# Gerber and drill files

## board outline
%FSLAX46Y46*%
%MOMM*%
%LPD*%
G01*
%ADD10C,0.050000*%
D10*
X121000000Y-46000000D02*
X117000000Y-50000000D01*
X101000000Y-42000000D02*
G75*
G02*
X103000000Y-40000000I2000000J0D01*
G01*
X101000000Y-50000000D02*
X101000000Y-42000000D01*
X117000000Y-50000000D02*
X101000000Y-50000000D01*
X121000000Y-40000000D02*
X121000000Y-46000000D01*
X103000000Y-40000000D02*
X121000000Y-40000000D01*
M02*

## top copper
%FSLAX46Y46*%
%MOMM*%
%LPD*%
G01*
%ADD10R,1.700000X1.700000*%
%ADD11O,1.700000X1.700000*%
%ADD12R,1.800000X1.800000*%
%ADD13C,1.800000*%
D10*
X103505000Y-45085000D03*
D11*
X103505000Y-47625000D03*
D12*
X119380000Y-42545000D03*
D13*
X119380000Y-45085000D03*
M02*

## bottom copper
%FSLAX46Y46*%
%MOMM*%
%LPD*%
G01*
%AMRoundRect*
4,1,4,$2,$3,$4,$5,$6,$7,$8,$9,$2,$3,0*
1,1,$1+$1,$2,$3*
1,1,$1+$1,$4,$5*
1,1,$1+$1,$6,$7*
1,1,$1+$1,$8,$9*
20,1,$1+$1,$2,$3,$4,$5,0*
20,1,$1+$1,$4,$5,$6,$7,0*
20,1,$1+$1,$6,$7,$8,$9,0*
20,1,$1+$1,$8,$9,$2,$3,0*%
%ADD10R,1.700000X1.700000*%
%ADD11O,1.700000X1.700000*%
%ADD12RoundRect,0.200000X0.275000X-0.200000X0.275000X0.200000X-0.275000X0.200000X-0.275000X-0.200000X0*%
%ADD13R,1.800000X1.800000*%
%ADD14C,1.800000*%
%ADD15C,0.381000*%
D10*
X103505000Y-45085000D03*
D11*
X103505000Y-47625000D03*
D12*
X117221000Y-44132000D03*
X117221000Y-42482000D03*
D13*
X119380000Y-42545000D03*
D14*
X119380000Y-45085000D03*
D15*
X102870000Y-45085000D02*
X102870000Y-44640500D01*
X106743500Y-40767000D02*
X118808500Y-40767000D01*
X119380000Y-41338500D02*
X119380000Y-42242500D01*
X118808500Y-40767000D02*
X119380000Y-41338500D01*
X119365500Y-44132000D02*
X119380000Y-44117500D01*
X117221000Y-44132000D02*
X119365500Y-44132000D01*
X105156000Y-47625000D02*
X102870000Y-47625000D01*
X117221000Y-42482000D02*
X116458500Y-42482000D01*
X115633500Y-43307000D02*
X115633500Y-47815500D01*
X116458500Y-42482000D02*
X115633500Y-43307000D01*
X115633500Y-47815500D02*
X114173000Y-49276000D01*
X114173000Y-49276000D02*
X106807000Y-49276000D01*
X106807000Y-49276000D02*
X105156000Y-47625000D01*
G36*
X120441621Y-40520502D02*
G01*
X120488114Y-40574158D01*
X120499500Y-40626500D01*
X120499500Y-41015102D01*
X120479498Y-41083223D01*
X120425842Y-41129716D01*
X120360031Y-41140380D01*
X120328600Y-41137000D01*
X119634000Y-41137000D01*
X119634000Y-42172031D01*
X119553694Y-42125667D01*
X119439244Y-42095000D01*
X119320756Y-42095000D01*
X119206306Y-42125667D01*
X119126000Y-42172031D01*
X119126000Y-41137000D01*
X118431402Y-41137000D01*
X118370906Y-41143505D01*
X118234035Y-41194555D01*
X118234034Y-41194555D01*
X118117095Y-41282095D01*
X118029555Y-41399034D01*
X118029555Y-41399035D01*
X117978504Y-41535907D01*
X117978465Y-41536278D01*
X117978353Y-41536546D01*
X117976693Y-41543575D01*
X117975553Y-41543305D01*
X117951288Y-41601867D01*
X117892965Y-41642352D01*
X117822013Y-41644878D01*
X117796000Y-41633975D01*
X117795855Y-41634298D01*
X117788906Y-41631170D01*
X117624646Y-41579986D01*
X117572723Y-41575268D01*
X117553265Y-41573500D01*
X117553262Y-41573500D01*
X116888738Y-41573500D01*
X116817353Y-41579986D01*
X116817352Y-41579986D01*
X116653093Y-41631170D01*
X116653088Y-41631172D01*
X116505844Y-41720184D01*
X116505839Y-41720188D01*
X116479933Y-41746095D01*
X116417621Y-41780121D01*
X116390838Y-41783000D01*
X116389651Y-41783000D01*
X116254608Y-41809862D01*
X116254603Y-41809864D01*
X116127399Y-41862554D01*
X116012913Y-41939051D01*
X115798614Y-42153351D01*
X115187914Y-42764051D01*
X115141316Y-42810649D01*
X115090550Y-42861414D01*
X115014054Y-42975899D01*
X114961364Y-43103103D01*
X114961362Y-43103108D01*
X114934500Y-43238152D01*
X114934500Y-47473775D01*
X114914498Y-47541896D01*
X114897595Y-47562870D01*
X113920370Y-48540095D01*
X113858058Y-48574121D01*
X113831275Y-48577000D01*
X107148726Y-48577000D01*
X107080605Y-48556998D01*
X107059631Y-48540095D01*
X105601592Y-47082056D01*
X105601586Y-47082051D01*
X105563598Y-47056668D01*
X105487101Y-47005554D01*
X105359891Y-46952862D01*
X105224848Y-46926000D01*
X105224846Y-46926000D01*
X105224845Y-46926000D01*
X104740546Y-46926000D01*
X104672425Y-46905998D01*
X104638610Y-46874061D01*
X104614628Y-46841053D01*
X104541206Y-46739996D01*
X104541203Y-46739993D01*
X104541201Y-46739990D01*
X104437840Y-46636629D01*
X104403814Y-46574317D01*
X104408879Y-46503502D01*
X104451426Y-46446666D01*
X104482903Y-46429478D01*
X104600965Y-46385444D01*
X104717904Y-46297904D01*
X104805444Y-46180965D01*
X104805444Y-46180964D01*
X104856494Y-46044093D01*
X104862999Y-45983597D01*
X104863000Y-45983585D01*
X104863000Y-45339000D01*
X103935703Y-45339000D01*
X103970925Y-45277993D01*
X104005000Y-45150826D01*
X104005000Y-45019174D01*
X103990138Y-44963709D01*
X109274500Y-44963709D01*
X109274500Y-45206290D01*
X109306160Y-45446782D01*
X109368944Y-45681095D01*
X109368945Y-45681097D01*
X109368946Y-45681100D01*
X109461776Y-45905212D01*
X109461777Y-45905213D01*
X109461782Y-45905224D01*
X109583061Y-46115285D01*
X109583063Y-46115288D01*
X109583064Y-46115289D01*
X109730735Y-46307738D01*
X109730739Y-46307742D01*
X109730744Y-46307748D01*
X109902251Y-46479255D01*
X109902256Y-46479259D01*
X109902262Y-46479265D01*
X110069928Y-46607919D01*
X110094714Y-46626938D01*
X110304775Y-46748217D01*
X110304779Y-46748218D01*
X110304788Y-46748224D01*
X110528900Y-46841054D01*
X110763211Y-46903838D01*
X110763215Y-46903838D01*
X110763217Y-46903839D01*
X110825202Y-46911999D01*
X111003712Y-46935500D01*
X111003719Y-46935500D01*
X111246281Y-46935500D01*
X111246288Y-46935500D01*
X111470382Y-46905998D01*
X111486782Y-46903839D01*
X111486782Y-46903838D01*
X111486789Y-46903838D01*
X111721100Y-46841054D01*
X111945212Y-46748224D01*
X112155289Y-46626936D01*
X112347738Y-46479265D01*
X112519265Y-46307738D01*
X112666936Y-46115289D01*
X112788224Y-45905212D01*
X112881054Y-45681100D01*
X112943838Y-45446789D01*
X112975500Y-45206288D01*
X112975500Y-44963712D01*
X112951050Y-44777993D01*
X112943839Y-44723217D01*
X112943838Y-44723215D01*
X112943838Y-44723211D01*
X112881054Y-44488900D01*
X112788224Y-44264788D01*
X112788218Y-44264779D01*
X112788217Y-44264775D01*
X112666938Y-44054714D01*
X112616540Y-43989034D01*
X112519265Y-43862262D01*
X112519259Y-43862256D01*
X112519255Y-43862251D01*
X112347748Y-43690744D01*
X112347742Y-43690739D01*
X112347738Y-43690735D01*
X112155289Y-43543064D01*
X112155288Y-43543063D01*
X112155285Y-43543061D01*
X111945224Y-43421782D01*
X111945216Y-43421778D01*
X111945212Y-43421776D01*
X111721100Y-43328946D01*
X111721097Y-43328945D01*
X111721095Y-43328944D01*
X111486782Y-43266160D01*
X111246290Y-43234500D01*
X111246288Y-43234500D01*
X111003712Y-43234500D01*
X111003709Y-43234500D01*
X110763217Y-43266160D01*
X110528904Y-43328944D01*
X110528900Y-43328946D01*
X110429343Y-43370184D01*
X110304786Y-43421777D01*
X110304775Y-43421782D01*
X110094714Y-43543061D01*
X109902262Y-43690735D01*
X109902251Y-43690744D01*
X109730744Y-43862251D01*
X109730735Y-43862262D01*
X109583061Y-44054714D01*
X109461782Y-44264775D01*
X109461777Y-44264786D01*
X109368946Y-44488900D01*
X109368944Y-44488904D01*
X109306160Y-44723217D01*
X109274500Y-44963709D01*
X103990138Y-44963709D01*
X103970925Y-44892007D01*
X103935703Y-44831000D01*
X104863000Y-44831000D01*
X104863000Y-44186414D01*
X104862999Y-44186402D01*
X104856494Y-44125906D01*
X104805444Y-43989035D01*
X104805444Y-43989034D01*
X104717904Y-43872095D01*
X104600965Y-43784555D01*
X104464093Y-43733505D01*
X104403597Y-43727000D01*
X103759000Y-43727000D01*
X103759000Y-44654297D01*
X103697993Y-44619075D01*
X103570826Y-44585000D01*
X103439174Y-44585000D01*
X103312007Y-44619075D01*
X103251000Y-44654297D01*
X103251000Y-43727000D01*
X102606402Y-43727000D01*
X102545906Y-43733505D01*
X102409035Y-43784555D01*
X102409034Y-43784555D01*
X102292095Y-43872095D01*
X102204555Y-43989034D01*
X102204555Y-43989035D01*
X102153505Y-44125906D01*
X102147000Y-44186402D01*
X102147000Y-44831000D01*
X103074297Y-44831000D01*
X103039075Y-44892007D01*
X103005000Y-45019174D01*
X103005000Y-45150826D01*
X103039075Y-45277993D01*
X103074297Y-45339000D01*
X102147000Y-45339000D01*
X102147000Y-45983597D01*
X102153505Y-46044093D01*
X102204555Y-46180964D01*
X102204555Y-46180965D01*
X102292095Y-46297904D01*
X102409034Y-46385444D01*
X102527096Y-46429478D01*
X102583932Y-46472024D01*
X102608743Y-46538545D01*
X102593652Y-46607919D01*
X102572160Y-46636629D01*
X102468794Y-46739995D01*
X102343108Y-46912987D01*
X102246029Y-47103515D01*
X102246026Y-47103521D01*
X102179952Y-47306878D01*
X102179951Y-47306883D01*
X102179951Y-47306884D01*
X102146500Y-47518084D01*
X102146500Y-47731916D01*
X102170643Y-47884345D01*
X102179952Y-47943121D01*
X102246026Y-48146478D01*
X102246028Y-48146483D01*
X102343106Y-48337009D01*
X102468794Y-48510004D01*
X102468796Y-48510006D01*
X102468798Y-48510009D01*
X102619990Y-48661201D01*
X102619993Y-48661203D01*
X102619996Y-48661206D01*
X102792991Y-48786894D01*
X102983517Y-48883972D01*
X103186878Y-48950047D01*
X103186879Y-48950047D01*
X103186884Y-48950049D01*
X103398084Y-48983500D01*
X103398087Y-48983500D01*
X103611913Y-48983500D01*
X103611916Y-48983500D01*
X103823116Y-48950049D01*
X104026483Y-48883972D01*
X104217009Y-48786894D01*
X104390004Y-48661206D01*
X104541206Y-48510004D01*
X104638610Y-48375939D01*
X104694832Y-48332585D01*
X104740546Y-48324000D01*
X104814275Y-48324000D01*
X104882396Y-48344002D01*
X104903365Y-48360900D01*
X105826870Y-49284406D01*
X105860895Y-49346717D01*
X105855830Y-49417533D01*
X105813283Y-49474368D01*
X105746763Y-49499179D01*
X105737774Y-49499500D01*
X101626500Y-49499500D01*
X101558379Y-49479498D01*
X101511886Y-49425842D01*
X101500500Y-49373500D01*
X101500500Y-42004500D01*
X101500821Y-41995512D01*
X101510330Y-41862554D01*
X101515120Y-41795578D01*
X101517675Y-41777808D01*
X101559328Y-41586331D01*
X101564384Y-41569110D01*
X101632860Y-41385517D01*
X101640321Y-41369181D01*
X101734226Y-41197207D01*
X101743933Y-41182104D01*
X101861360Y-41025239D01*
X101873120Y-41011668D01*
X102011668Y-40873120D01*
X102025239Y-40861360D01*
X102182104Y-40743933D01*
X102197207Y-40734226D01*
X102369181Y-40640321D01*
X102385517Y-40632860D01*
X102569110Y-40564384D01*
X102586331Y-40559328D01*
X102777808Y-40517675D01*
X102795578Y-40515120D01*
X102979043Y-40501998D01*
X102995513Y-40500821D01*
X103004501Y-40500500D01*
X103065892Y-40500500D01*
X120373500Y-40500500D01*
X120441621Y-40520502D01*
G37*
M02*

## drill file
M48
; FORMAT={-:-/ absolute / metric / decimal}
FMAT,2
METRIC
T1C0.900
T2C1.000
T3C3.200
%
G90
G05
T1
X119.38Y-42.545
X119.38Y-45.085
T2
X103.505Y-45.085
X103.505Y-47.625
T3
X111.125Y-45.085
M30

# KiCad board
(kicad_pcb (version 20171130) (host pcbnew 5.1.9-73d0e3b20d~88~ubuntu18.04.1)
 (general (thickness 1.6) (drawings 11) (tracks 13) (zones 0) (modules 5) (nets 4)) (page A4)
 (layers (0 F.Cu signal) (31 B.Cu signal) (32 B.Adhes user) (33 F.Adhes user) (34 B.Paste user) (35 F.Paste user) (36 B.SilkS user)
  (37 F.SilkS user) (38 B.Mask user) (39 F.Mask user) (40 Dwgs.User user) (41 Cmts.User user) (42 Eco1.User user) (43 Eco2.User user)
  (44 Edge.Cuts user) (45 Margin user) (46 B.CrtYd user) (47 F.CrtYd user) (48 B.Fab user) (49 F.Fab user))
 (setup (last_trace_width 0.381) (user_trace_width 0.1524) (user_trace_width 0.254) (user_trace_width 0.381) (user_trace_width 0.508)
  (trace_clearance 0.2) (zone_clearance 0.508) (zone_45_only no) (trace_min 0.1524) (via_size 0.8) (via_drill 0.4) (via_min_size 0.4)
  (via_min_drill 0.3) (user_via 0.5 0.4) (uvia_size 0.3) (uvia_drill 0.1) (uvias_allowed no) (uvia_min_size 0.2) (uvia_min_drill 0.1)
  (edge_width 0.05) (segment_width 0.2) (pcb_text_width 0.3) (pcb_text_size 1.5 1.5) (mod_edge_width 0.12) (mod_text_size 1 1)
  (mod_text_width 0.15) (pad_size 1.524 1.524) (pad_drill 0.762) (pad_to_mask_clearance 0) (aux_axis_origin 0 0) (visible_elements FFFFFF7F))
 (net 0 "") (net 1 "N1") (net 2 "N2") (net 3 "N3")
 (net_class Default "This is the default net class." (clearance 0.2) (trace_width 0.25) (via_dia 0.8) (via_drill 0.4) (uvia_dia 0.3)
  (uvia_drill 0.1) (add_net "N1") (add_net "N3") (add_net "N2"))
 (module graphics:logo (layer F.Cu) (at 118 43)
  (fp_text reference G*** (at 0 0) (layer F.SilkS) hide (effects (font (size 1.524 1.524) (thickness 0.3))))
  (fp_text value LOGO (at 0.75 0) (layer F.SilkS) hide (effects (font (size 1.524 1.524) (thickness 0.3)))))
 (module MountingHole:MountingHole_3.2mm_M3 (layer F.Cu) (at 111.125 45.085)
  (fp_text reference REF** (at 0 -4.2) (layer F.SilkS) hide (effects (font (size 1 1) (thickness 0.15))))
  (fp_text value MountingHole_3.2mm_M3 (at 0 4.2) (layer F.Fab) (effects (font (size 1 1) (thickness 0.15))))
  (pad 1 np_thru_hole circle (at 0 0) (size 3.2 3.2) (drill 3.2) (layers *.Cu *.Mask)))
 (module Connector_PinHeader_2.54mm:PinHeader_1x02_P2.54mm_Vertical (layer F.Cu) (at 103.505 45.085)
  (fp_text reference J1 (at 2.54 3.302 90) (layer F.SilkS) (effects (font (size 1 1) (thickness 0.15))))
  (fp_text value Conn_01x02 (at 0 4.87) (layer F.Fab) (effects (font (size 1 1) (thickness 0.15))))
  (pad 1 thru_hole rect (at 0 0) (size 1.7 1.7) (drill 1) (layers *.Cu *.Mask) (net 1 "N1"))
  (pad 2 thru_hole oval (at 0 2.54) (size 1.7 1.7) (drill 1) (layers *.Cu *.Mask) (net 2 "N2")))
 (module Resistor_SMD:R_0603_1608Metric (layer B.Cu) (at 117.221 43.307 90)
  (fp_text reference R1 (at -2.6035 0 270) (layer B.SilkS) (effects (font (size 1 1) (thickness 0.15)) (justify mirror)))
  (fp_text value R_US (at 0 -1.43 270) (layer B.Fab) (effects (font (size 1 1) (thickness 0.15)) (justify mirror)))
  (pad 1 smd roundrect (at -0.825 0 90) (size 0.8 0.95) (layers B.Cu B.Paste B.Mask) (roundrect_rratio 0.25) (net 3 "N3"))
  (pad 2 smd roundrect (at 0.825 0 90) (size 0.8 0.95) (layers B.Cu B.Paste B.Mask) (roundrect_rratio 0.25) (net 2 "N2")))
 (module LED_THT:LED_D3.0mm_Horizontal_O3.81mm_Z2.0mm (layer B.Cu) (at 119.38 42.545 270)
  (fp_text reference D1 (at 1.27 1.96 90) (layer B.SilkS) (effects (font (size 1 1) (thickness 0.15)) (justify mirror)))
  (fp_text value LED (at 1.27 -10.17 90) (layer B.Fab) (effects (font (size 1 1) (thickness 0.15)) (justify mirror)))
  (pad 1 thru_hole rect (at 0 0 270) (size 1.8 1.8) (drill 0.9) (layers *.Cu *.Mask) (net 1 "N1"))
  (pad 2 thru_hole circle (at 2.54 0 270) (size 1.8 1.8) (drill 0.9) (layers *.Cu *.Mask) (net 3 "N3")))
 (gr_line (start 121 46) (end 117 50) (layer Edge.Cuts) (width 0.05))
 (gr_arc (start 103 42) (end 103 40) (angle -90) (layer Edge.Cuts) (width 0.05))
 (gr_line (start 101 50) (end 101 42) (layer Edge.Cuts) (width 0.05))
 (gr_line (start 117 50) (end 101 50) (layer Edge.Cuts) (width 0.05))
 (gr_line (start 121 40) (end 121 46) (layer Edge.Cuts) (width 0.05))
 (gr_line (start 103 40) (end 121 40) (layer Edge.Cuts) (width 0.05))
 (segment (start 102.87 45.085) (end 102.87 44.6405) (width 0.381) (layer B.Cu) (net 1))
 (segment (start 106.7435 40.767) (end 118.8085 40.767) (width 0.381) (layer B.Cu) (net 1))
 (segment (start 119.38 41.3385) (end 119.38 42.2425) (width 0.381) (layer B.Cu) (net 1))
 (segment (start 118.8085 40.767) (end 119.38 41.3385) (width 0.381) (layer B.Cu) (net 1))
 (segment (start 119.3655 44.132) (end 119.38 44.1175) (width 0.381) (layer B.Cu) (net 3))
 (segment (start 117.221 44.132) (end 119.3655 44.132) (width 0.381) (layer B.Cu) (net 3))
 (segment (start 105.156 47.625) (end 102.87 47.625) (width 0.381) (layer B.Cu) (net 2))
 (segment (start 117.221 42.482) (end 116.4585 42.482) (width 0.381) (layer B.Cu) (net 2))
 (segment (start 115.6335 43.307) (end 115.6335 47.8155) (width 0.381) (layer B.Cu) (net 2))
 (segment (start 116.4585 42.482) (end 115.6335 43.307) (width 0.381) (layer B.Cu) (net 2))
 (segment (start 115.6335 47.8155) (end 114.173 49.276) (width 0.381) (layer B.Cu) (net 2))
 (segment (start 114.173 49.276) (end 106.807 49.276) (width 0.381) (layer B.Cu) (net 2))
 (segment (start 106.807 49.276) (end 105.156 47.625) (width 0.381) (layer B.Cu) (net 2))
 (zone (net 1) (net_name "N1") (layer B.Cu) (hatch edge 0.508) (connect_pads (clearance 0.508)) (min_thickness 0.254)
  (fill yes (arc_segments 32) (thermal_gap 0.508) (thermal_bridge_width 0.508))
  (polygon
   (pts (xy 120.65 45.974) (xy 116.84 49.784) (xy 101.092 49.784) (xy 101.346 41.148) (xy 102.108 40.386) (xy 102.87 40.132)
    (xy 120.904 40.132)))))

